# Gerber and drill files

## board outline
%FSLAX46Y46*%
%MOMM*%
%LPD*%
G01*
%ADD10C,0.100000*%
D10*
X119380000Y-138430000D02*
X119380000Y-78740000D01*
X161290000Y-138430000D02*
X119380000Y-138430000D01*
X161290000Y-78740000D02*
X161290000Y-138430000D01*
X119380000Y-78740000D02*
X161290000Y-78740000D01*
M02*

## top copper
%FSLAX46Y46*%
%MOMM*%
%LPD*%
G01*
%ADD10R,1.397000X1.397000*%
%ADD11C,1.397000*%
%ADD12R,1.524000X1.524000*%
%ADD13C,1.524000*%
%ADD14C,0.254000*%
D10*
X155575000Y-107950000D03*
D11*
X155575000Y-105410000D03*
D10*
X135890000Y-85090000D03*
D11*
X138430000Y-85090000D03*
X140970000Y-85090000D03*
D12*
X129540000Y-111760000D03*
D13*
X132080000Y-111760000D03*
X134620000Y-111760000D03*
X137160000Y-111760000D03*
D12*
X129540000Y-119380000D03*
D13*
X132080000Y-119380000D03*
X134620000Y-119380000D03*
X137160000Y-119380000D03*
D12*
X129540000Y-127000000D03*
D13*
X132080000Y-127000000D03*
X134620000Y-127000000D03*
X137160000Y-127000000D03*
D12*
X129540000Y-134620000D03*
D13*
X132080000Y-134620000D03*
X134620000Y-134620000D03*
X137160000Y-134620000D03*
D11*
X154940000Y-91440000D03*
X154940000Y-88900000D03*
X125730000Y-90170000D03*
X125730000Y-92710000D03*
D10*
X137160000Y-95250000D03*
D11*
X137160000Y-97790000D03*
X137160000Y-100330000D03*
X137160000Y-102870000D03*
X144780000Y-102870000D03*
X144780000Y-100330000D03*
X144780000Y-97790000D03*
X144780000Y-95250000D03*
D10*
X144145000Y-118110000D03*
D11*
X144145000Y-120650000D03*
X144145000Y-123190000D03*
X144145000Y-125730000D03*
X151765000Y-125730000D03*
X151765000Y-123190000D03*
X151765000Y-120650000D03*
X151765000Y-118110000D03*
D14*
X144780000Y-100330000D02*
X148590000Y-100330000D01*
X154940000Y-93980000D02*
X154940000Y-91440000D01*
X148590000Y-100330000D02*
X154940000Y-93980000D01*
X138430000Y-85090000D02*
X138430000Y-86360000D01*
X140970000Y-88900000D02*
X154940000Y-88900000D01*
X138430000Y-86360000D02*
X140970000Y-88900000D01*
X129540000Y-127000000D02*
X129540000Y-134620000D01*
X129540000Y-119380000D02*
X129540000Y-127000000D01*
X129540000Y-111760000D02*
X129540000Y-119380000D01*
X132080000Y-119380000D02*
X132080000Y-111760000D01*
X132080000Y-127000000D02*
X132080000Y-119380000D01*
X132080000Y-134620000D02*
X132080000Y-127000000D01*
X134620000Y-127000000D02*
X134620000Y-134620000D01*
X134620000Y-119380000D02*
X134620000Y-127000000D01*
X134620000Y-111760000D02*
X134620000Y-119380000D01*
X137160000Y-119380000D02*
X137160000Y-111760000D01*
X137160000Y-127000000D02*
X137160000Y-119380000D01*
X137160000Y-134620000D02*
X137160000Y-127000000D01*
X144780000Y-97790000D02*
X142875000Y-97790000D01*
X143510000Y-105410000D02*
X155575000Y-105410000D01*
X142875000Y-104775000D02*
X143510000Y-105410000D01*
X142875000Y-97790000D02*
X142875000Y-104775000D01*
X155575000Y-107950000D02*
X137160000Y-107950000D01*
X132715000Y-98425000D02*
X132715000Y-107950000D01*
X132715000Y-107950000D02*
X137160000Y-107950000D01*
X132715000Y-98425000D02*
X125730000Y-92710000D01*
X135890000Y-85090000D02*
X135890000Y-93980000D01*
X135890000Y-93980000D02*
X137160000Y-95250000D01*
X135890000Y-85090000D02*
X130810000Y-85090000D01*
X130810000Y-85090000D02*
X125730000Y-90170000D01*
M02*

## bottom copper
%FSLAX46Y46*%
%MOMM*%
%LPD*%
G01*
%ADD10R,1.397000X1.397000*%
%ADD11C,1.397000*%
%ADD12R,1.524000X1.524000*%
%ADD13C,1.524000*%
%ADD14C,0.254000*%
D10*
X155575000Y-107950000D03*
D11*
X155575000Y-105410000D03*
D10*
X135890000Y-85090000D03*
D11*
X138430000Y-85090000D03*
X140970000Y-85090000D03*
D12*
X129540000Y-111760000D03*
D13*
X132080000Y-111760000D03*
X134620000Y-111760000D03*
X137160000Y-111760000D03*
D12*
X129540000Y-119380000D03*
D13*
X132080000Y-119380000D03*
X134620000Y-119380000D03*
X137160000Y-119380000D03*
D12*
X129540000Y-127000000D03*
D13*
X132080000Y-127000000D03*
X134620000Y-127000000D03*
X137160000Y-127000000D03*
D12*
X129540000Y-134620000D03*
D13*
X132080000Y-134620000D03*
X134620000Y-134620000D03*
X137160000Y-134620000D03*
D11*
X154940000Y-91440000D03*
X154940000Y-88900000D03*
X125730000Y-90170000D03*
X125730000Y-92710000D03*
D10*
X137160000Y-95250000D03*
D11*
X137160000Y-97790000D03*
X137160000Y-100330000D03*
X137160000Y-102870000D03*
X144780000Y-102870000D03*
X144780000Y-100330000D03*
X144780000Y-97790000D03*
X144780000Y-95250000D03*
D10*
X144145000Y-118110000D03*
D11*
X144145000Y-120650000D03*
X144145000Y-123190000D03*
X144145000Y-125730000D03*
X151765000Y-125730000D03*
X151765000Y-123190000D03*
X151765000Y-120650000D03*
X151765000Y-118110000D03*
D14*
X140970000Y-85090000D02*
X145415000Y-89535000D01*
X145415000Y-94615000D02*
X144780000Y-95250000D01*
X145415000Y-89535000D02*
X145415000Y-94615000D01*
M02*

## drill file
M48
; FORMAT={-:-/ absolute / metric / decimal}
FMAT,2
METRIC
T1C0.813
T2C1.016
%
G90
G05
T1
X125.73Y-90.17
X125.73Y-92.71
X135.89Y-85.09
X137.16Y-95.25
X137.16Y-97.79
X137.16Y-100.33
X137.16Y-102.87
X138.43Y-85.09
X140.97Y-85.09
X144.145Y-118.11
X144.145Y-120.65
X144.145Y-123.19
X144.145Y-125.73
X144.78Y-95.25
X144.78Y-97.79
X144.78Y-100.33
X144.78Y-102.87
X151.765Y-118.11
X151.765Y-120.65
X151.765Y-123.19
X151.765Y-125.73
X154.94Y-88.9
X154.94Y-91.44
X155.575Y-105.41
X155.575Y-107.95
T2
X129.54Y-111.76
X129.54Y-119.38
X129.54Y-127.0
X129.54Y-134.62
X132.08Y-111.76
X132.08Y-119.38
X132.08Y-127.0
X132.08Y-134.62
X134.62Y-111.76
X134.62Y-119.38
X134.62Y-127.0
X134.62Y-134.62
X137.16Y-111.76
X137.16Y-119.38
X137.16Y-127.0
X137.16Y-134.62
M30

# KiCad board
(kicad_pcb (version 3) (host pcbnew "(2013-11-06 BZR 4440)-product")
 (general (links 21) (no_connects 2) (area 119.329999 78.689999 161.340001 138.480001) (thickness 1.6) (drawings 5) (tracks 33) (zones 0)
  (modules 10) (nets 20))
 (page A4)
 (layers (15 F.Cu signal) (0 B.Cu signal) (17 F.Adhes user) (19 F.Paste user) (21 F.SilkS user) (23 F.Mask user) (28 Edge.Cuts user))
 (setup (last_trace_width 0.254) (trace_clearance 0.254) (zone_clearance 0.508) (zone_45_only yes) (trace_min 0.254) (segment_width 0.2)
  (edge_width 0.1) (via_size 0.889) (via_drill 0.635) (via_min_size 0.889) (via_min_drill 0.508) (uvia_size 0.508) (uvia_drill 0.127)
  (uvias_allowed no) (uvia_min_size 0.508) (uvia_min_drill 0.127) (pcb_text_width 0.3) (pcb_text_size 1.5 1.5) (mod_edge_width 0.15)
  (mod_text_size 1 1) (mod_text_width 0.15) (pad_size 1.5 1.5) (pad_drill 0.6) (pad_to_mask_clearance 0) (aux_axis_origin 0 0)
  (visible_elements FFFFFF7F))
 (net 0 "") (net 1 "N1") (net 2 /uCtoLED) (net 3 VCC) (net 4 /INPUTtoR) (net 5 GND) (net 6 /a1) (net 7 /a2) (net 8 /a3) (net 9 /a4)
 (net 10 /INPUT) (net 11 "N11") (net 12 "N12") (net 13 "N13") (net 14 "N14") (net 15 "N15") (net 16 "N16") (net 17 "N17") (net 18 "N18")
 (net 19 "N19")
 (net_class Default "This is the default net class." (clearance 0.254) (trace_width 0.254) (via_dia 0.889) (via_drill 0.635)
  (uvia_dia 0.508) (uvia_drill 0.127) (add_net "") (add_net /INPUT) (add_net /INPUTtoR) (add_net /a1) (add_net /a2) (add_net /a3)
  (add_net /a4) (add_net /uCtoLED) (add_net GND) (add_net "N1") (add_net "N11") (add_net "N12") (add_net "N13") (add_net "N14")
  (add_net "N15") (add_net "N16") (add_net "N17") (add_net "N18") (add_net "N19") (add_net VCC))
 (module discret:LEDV (layer F.Cu) (at 155.575 106.68 90)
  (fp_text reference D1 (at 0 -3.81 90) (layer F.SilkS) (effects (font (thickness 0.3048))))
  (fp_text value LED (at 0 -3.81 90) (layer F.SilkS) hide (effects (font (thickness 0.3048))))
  (pad 1 thru_hole rect (at -1.27 0 90) (size 1.397 1.397) (drill 0.8128) (layers *.Cu *.Mask F.SilkS) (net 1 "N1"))
  (pad 2 thru_hole circle (at 1.27 0 90) (size 1.397 1.397) (drill 0.8128) (layers *.Cu *.Mask F.SilkS) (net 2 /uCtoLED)))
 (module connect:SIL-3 (layer F.Cu) (at 138.43 85.09)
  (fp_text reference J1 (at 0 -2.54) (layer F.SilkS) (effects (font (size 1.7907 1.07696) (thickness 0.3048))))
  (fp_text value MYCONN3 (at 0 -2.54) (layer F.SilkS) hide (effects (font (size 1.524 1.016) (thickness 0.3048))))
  (pad 1 thru_hole rect (at -2.54 0) (size 1.397 1.397) (drill 0.8128) (layers *.Cu *.Mask F.SilkS) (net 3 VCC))
  (pad 2 thru_hole circle (at 0 0) (size 1.397 1.397) (drill 0.8128) (layers *.Cu *.Mask F.SilkS) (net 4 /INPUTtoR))
  (pad 3 thru_hole circle (at 2.54 0) (size 1.397 1.397) (drill 0.8128) (layers *.Cu *.Mask F.SilkS) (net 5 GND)))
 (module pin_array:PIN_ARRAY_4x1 (layer F.Cu) (at 133.35 111.76)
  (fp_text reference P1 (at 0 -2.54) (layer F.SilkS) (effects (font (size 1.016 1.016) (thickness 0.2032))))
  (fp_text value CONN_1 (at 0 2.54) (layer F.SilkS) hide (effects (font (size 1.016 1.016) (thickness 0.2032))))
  (pad 1 thru_hole rect (at -3.81 0) (size 1.524 1.524) (drill 1.016) (layers *.Cu *.Mask F.SilkS) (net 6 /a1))
  (pad 2 thru_hole circle (at -1.27 0) (size 1.524 1.524) (drill 1.016) (layers *.Cu *.Mask F.SilkS) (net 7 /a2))
  (pad 3 thru_hole circle (at 1.27 0) (size 1.524 1.524) (drill 1.016) (layers *.Cu *.Mask F.SilkS) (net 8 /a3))
  (pad 4 thru_hole circle (at 3.81 0) (size 1.524 1.524) (drill 1.016) (layers *.Cu *.Mask F.SilkS) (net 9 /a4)))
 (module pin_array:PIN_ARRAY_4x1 (layer F.Cu) (at 133.35 119.38)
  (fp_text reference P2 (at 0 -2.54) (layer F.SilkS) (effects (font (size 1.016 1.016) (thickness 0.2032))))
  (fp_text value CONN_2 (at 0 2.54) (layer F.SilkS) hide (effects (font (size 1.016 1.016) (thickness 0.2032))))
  (pad 1 thru_hole rect (at -3.81 0) (size 1.524 1.524) (drill 1.016) (layers *.Cu *.Mask F.SilkS) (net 6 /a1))
  (pad 2 thru_hole circle (at -1.27 0) (size 1.524 1.524) (drill 1.016) (layers *.Cu *.Mask F.SilkS) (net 7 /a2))
  (pad 3 thru_hole circle (at 1.27 0) (size 1.524 1.524) (drill 1.016) (layers *.Cu *.Mask F.SilkS) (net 8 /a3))
  (pad 4 thru_hole circle (at 3.81 0) (size 1.524 1.524) (drill 1.016) (layers *.Cu *.Mask F.SilkS) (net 9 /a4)))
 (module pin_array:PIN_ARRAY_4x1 (layer F.Cu) (at 133.35 127)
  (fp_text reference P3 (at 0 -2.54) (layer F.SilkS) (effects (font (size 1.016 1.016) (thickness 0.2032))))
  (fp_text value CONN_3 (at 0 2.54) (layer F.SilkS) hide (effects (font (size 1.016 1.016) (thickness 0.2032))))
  (pad 1 thru_hole rect (at -3.81 0) (size 1.524 1.524) (drill 1.016) (layers *.Cu *.Mask F.SilkS) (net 6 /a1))
  (pad 2 thru_hole circle (at -1.27 0) (size 1.524 1.524) (drill 1.016) (layers *.Cu *.Mask F.SilkS) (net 7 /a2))
  (pad 3 thru_hole circle (at 1.27 0) (size 1.524 1.524) (drill 1.016) (layers *.Cu *.Mask F.SilkS) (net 8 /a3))
  (pad 4 thru_hole circle (at 3.81 0) (size 1.524 1.524) (drill 1.016) (layers *.Cu *.Mask F.SilkS) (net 9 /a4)))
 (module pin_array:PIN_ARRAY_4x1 (layer F.Cu) (at 133.35 134.62)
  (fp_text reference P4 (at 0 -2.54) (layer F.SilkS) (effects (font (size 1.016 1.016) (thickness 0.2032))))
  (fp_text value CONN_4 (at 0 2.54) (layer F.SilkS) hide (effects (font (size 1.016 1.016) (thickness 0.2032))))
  (pad 1 thru_hole rect (at -3.81 0) (size 1.524 1.524) (drill 1.016) (layers *.Cu *.Mask F.SilkS) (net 6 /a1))
  (pad 2 thru_hole circle (at -1.27 0) (size 1.524 1.524) (drill 1.016) (layers *.Cu *.Mask F.SilkS) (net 7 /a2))
  (pad 3 thru_hole circle (at 1.27 0) (size 1.524 1.524) (drill 1.016) (layers *.Cu *.Mask F.SilkS) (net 8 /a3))
  (pad 4 thru_hole circle (at 3.81 0) (size 1.524 1.524) (drill 1.016) (layers *.Cu *.Mask F.SilkS) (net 9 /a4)))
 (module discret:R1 (layer F.Cu) (at 154.94 90.17 90) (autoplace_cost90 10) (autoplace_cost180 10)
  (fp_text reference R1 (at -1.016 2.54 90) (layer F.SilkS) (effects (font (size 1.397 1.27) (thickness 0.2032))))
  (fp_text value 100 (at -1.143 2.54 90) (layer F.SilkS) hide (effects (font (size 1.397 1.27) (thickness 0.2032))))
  (pad 1 thru_hole circle (at -1.27 0 90) (size 1.397 1.397) (drill 0.8128) (layers *.Cu *.Mask F.SilkS) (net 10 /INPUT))
  (pad 2 thru_hole circle (at 1.27 0 90) (size 1.397 1.397) (drill 0.8128) (layers *.Cu *.Mask F.SilkS) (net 4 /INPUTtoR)))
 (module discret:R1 (layer F.Cu) (at 125.73 91.44 270) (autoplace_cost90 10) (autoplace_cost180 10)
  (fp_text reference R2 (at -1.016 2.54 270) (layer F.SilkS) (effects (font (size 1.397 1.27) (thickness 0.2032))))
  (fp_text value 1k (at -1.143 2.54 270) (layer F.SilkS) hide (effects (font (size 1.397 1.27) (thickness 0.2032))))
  (pad 1 thru_hole circle (at -1.27 0 270) (size 1.397 1.397) (drill 0.8128) (layers *.Cu *.Mask F.SilkS) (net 3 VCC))
  (pad 2 thru_hole circle (at 1.27 0 270) (size 1.397 1.397) (drill 0.8128) (layers *.Cu *.Mask F.SilkS) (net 1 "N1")))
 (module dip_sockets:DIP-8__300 (layer F.Cu) (at 140.97 99.06 270)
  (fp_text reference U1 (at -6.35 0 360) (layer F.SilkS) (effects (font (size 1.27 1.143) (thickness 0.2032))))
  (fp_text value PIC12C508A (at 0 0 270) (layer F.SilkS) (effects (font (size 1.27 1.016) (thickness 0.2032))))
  (pad 1 thru_hole rect (at -3.81 3.81 270) (size 1.397 1.397) (drill 0.8128) (layers *.Cu *.Mask F.SilkS) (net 3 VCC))
  (pad 2 thru_hole circle (at -1.27 3.81 270) (size 1.397 1.397) (drill 0.8128) (layers *.Cu *.Mask F.SilkS) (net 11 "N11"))
  (pad 3 thru_hole circle (at 1.27 3.81 270) (size 1.397 1.397) (drill 0.8128) (layers *.Cu *.Mask F.SilkS) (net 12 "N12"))
  (pad 4 thru_hole circle (at 3.81 3.81 270) (size 1.397 1.397) (drill 0.8128) (layers *.Cu *.Mask F.SilkS) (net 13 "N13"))
  (pad 5 thru_hole circle (at 3.81 -3.81 270) (size 1.397 1.397) (drill 0.8128) (layers *.Cu *.Mask F.SilkS) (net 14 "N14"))
  (pad 6 thru_hole circle (at 1.27 -3.81 270) (size 1.397 1.397) (drill 0.8128) (layers *.Cu *.Mask F.SilkS) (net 10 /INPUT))
  (pad 7 thru_hole circle (at -1.27 -3.81 270) (size 1.397 1.397) (drill 0.8128) (layers *.Cu *.Mask F.SilkS) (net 2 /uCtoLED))
  (pad 8 thru_hole circle (at -3.81 -3.81 270) (size 1.397 1.397) (drill 0.8128) (layers *.Cu *.Mask F.SilkS) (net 5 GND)))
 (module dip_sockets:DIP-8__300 (layer F.Cu) (at 147.955 121.92 270)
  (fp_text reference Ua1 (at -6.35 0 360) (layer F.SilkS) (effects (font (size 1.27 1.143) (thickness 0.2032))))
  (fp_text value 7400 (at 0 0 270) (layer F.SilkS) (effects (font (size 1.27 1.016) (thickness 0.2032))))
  (pad 1 thru_hole rect (at -3.81 3.81 270) (size 1.397 1.397) (drill 0.8128) (layers *.Cu *.Mask F.SilkS) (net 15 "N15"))
  (pad 2 thru_hole circle (at -1.27 3.81 270) (size 1.397 1.397) (drill 0.8128) (layers *.Cu *.Mask F.SilkS) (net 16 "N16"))
  (pad 3 thru_hole circle (at 1.27 3.81 270) (size 1.397 1.397) (drill 0.8128) (layers *.Cu *.Mask F.SilkS) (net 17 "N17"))
  (pad 4 thru_hole circle (at 3.81 3.81 270) (size 1.397 1.397) (drill 0.8128) (layers *.Cu *.Mask F.SilkS) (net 17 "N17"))
  (pad 5 thru_hole circle (at 3.81 -3.81 270) (size 1.397 1.397) (drill 0.8128) (layers *.Cu *.Mask F.SilkS) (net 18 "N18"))
  (pad 6 thru_hole circle (at 1.27 -3.81 270) (size 1.397 1.397) (drill 0.8128) (layers *.Cu *.Mask F.SilkS) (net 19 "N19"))
  (pad 7 thru_hole circle (at -1.27 -3.81 270) (size 1.397 1.397) (drill 0.8128) (layers *.Cu *.Mask F.SilkS) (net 5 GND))
  (pad 8 thru_hole circle (at -3.81 -3.81 270) (size 1.397 1.397) (drill 0.8128) (layers *.Cu *.Mask F.SilkS)))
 (gr_line (start 119.38 138.43) (end 119.38 78.74) (angle 90) (layer Edge.Cuts) (width 0.1))
 (gr_line (start 161.29 138.43) (end 119.38 138.43) (angle 90) (layer Edge.Cuts) (width 0.1))
 (gr_line (start 161.29 78.74) (end 161.29 138.43) (angle 90) (layer Edge.Cuts) (width 0.1))
 (gr_line (start 119.38 78.74) (end 161.29 78.74) (angle 90) (layer Edge.Cuts) (width 0.1))
 (segment (start 144.78 100.33) (end 148.59 100.33) (width 0.254) (layer F.Cu) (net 10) (status 10))
 (segment (start 154.94 93.98) (end 154.94 91.44) (width 0.254) (layer F.Cu) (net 10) (status 20))
 (segment (start 148.59 100.33) (end 154.94 93.98) (width 0.254) (layer F.Cu) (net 10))
 (segment (start 138.43 85.09) (end 138.43 86.36) (width 0.254) (layer F.Cu) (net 4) (status 10))
 (segment (start 140.97 88.9) (end 154.94 88.9) (width 0.254) (layer F.Cu) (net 4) (status 20))
 (segment (start 138.43 86.36) (end 140.97 88.9) (width 0.254) (layer F.Cu) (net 4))
 (segment (start 129.54 127) (end 129.54 134.62) (width 0.254) (layer F.Cu) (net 6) (status 30))
 (segment (start 129.54 119.38) (end 129.54 127) (width 0.254) (layer F.Cu) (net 6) (status 30))
 (segment (start 129.54 111.76) (end 129.54 119.38) (width 0.254) (layer F.Cu) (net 6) (status 30))
 (segment (start 132.08 119.38) (end 132.08 111.76) (width 0.254) (layer F.Cu) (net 7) (status 30))
 (segment (start 132.08 127) (end 132.08 119.38) (width 0.254) (layer F.Cu) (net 7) (status 30))
 (segment (start 132.08 134.62) (end 132.08 127) (width 0.254) (layer F.Cu) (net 7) (status 30))
 (segment (start 134.62 127) (end 134.62 134.62) (width 0.254) (layer F.Cu) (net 8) (status 30))
 (segment (start 134.62 119.38) (end 134.62 127) (width 0.254) (layer F.Cu) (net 8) (status 30))
 (segment (start 134.62 111.76) (end 134.62 119.38) (width 0.254) (layer F.Cu) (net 8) (status 30))
 (segment (start 137.16 119.38) (end 137.16 111.76) (width 0.254) (layer F.Cu) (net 9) (status 30))
 (segment (start 137.16 127) (end 137.16 119.38) (width 0.254) (layer F.Cu) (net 9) (status 30))
 (segment (start 137.16 134.62) (end 137.16 127) (width 0.254) (layer F.Cu) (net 9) (status 30))
 (segment (start 144.78 97.79) (end 142.875 97.79) (width 0.254) (layer F.Cu) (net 2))
 (segment (start 143.51 105.41) (end 155.575 105.41) (width 0.254) (layer F.Cu) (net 2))
 (segment (start 142.875 104.775) (end 143.51 105.41) (width 0.254) (layer F.Cu) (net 2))
 (segment (start 142.875 97.79) (end 142.875 104.775) (width 0.254) (layer F.Cu) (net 2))
 (segment (start 140.97 85.09) (end 145.415 89.535) (width 0.254) (layer B.Cu) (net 5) (status 10))
 (segment (start 145.415 94.615) (end 144.78 95.25) (width 0.254) (layer B.Cu) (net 5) (status 20))
 (segment (start 145.415 89.535) (end 145.415 94.615) (width 0.254) (layer B.Cu) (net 5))
 (segment (start 155.575 107.95) (end 137.16 107.95) (width 0.254) (layer F.Cu) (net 1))
 (segment (start 132.715 98.425) (end 132.715 107.95) (width 0.254) (layer F.Cu) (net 1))
 (segment (start 132.715 107.95) (end 137.16 107.95) (width 0.254) (layer F.Cu) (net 1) (status 20))
 (segment (start 132.715 98.425) (end 125.73 92.71) (width 0.254) (layer F.Cu) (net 1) (status 10))
 (segment (start 135.89 85.09) (end 135.89 93.98) (width 0.254) (layer F.Cu) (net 3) (status 10))
 (segment (start 135.89 93.98) (end 137.16 95.25) (width 0.254) (layer F.Cu) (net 3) (status 20))
 (segment (start 135.89 85.09) (end 130.81 85.09) (width 0.254) (layer F.Cu) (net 3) (status 10))
 (segment (start 130.81 85.09) (end 125.73 90.17) (width 0.254) (layer F.Cu) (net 3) (status 20)))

